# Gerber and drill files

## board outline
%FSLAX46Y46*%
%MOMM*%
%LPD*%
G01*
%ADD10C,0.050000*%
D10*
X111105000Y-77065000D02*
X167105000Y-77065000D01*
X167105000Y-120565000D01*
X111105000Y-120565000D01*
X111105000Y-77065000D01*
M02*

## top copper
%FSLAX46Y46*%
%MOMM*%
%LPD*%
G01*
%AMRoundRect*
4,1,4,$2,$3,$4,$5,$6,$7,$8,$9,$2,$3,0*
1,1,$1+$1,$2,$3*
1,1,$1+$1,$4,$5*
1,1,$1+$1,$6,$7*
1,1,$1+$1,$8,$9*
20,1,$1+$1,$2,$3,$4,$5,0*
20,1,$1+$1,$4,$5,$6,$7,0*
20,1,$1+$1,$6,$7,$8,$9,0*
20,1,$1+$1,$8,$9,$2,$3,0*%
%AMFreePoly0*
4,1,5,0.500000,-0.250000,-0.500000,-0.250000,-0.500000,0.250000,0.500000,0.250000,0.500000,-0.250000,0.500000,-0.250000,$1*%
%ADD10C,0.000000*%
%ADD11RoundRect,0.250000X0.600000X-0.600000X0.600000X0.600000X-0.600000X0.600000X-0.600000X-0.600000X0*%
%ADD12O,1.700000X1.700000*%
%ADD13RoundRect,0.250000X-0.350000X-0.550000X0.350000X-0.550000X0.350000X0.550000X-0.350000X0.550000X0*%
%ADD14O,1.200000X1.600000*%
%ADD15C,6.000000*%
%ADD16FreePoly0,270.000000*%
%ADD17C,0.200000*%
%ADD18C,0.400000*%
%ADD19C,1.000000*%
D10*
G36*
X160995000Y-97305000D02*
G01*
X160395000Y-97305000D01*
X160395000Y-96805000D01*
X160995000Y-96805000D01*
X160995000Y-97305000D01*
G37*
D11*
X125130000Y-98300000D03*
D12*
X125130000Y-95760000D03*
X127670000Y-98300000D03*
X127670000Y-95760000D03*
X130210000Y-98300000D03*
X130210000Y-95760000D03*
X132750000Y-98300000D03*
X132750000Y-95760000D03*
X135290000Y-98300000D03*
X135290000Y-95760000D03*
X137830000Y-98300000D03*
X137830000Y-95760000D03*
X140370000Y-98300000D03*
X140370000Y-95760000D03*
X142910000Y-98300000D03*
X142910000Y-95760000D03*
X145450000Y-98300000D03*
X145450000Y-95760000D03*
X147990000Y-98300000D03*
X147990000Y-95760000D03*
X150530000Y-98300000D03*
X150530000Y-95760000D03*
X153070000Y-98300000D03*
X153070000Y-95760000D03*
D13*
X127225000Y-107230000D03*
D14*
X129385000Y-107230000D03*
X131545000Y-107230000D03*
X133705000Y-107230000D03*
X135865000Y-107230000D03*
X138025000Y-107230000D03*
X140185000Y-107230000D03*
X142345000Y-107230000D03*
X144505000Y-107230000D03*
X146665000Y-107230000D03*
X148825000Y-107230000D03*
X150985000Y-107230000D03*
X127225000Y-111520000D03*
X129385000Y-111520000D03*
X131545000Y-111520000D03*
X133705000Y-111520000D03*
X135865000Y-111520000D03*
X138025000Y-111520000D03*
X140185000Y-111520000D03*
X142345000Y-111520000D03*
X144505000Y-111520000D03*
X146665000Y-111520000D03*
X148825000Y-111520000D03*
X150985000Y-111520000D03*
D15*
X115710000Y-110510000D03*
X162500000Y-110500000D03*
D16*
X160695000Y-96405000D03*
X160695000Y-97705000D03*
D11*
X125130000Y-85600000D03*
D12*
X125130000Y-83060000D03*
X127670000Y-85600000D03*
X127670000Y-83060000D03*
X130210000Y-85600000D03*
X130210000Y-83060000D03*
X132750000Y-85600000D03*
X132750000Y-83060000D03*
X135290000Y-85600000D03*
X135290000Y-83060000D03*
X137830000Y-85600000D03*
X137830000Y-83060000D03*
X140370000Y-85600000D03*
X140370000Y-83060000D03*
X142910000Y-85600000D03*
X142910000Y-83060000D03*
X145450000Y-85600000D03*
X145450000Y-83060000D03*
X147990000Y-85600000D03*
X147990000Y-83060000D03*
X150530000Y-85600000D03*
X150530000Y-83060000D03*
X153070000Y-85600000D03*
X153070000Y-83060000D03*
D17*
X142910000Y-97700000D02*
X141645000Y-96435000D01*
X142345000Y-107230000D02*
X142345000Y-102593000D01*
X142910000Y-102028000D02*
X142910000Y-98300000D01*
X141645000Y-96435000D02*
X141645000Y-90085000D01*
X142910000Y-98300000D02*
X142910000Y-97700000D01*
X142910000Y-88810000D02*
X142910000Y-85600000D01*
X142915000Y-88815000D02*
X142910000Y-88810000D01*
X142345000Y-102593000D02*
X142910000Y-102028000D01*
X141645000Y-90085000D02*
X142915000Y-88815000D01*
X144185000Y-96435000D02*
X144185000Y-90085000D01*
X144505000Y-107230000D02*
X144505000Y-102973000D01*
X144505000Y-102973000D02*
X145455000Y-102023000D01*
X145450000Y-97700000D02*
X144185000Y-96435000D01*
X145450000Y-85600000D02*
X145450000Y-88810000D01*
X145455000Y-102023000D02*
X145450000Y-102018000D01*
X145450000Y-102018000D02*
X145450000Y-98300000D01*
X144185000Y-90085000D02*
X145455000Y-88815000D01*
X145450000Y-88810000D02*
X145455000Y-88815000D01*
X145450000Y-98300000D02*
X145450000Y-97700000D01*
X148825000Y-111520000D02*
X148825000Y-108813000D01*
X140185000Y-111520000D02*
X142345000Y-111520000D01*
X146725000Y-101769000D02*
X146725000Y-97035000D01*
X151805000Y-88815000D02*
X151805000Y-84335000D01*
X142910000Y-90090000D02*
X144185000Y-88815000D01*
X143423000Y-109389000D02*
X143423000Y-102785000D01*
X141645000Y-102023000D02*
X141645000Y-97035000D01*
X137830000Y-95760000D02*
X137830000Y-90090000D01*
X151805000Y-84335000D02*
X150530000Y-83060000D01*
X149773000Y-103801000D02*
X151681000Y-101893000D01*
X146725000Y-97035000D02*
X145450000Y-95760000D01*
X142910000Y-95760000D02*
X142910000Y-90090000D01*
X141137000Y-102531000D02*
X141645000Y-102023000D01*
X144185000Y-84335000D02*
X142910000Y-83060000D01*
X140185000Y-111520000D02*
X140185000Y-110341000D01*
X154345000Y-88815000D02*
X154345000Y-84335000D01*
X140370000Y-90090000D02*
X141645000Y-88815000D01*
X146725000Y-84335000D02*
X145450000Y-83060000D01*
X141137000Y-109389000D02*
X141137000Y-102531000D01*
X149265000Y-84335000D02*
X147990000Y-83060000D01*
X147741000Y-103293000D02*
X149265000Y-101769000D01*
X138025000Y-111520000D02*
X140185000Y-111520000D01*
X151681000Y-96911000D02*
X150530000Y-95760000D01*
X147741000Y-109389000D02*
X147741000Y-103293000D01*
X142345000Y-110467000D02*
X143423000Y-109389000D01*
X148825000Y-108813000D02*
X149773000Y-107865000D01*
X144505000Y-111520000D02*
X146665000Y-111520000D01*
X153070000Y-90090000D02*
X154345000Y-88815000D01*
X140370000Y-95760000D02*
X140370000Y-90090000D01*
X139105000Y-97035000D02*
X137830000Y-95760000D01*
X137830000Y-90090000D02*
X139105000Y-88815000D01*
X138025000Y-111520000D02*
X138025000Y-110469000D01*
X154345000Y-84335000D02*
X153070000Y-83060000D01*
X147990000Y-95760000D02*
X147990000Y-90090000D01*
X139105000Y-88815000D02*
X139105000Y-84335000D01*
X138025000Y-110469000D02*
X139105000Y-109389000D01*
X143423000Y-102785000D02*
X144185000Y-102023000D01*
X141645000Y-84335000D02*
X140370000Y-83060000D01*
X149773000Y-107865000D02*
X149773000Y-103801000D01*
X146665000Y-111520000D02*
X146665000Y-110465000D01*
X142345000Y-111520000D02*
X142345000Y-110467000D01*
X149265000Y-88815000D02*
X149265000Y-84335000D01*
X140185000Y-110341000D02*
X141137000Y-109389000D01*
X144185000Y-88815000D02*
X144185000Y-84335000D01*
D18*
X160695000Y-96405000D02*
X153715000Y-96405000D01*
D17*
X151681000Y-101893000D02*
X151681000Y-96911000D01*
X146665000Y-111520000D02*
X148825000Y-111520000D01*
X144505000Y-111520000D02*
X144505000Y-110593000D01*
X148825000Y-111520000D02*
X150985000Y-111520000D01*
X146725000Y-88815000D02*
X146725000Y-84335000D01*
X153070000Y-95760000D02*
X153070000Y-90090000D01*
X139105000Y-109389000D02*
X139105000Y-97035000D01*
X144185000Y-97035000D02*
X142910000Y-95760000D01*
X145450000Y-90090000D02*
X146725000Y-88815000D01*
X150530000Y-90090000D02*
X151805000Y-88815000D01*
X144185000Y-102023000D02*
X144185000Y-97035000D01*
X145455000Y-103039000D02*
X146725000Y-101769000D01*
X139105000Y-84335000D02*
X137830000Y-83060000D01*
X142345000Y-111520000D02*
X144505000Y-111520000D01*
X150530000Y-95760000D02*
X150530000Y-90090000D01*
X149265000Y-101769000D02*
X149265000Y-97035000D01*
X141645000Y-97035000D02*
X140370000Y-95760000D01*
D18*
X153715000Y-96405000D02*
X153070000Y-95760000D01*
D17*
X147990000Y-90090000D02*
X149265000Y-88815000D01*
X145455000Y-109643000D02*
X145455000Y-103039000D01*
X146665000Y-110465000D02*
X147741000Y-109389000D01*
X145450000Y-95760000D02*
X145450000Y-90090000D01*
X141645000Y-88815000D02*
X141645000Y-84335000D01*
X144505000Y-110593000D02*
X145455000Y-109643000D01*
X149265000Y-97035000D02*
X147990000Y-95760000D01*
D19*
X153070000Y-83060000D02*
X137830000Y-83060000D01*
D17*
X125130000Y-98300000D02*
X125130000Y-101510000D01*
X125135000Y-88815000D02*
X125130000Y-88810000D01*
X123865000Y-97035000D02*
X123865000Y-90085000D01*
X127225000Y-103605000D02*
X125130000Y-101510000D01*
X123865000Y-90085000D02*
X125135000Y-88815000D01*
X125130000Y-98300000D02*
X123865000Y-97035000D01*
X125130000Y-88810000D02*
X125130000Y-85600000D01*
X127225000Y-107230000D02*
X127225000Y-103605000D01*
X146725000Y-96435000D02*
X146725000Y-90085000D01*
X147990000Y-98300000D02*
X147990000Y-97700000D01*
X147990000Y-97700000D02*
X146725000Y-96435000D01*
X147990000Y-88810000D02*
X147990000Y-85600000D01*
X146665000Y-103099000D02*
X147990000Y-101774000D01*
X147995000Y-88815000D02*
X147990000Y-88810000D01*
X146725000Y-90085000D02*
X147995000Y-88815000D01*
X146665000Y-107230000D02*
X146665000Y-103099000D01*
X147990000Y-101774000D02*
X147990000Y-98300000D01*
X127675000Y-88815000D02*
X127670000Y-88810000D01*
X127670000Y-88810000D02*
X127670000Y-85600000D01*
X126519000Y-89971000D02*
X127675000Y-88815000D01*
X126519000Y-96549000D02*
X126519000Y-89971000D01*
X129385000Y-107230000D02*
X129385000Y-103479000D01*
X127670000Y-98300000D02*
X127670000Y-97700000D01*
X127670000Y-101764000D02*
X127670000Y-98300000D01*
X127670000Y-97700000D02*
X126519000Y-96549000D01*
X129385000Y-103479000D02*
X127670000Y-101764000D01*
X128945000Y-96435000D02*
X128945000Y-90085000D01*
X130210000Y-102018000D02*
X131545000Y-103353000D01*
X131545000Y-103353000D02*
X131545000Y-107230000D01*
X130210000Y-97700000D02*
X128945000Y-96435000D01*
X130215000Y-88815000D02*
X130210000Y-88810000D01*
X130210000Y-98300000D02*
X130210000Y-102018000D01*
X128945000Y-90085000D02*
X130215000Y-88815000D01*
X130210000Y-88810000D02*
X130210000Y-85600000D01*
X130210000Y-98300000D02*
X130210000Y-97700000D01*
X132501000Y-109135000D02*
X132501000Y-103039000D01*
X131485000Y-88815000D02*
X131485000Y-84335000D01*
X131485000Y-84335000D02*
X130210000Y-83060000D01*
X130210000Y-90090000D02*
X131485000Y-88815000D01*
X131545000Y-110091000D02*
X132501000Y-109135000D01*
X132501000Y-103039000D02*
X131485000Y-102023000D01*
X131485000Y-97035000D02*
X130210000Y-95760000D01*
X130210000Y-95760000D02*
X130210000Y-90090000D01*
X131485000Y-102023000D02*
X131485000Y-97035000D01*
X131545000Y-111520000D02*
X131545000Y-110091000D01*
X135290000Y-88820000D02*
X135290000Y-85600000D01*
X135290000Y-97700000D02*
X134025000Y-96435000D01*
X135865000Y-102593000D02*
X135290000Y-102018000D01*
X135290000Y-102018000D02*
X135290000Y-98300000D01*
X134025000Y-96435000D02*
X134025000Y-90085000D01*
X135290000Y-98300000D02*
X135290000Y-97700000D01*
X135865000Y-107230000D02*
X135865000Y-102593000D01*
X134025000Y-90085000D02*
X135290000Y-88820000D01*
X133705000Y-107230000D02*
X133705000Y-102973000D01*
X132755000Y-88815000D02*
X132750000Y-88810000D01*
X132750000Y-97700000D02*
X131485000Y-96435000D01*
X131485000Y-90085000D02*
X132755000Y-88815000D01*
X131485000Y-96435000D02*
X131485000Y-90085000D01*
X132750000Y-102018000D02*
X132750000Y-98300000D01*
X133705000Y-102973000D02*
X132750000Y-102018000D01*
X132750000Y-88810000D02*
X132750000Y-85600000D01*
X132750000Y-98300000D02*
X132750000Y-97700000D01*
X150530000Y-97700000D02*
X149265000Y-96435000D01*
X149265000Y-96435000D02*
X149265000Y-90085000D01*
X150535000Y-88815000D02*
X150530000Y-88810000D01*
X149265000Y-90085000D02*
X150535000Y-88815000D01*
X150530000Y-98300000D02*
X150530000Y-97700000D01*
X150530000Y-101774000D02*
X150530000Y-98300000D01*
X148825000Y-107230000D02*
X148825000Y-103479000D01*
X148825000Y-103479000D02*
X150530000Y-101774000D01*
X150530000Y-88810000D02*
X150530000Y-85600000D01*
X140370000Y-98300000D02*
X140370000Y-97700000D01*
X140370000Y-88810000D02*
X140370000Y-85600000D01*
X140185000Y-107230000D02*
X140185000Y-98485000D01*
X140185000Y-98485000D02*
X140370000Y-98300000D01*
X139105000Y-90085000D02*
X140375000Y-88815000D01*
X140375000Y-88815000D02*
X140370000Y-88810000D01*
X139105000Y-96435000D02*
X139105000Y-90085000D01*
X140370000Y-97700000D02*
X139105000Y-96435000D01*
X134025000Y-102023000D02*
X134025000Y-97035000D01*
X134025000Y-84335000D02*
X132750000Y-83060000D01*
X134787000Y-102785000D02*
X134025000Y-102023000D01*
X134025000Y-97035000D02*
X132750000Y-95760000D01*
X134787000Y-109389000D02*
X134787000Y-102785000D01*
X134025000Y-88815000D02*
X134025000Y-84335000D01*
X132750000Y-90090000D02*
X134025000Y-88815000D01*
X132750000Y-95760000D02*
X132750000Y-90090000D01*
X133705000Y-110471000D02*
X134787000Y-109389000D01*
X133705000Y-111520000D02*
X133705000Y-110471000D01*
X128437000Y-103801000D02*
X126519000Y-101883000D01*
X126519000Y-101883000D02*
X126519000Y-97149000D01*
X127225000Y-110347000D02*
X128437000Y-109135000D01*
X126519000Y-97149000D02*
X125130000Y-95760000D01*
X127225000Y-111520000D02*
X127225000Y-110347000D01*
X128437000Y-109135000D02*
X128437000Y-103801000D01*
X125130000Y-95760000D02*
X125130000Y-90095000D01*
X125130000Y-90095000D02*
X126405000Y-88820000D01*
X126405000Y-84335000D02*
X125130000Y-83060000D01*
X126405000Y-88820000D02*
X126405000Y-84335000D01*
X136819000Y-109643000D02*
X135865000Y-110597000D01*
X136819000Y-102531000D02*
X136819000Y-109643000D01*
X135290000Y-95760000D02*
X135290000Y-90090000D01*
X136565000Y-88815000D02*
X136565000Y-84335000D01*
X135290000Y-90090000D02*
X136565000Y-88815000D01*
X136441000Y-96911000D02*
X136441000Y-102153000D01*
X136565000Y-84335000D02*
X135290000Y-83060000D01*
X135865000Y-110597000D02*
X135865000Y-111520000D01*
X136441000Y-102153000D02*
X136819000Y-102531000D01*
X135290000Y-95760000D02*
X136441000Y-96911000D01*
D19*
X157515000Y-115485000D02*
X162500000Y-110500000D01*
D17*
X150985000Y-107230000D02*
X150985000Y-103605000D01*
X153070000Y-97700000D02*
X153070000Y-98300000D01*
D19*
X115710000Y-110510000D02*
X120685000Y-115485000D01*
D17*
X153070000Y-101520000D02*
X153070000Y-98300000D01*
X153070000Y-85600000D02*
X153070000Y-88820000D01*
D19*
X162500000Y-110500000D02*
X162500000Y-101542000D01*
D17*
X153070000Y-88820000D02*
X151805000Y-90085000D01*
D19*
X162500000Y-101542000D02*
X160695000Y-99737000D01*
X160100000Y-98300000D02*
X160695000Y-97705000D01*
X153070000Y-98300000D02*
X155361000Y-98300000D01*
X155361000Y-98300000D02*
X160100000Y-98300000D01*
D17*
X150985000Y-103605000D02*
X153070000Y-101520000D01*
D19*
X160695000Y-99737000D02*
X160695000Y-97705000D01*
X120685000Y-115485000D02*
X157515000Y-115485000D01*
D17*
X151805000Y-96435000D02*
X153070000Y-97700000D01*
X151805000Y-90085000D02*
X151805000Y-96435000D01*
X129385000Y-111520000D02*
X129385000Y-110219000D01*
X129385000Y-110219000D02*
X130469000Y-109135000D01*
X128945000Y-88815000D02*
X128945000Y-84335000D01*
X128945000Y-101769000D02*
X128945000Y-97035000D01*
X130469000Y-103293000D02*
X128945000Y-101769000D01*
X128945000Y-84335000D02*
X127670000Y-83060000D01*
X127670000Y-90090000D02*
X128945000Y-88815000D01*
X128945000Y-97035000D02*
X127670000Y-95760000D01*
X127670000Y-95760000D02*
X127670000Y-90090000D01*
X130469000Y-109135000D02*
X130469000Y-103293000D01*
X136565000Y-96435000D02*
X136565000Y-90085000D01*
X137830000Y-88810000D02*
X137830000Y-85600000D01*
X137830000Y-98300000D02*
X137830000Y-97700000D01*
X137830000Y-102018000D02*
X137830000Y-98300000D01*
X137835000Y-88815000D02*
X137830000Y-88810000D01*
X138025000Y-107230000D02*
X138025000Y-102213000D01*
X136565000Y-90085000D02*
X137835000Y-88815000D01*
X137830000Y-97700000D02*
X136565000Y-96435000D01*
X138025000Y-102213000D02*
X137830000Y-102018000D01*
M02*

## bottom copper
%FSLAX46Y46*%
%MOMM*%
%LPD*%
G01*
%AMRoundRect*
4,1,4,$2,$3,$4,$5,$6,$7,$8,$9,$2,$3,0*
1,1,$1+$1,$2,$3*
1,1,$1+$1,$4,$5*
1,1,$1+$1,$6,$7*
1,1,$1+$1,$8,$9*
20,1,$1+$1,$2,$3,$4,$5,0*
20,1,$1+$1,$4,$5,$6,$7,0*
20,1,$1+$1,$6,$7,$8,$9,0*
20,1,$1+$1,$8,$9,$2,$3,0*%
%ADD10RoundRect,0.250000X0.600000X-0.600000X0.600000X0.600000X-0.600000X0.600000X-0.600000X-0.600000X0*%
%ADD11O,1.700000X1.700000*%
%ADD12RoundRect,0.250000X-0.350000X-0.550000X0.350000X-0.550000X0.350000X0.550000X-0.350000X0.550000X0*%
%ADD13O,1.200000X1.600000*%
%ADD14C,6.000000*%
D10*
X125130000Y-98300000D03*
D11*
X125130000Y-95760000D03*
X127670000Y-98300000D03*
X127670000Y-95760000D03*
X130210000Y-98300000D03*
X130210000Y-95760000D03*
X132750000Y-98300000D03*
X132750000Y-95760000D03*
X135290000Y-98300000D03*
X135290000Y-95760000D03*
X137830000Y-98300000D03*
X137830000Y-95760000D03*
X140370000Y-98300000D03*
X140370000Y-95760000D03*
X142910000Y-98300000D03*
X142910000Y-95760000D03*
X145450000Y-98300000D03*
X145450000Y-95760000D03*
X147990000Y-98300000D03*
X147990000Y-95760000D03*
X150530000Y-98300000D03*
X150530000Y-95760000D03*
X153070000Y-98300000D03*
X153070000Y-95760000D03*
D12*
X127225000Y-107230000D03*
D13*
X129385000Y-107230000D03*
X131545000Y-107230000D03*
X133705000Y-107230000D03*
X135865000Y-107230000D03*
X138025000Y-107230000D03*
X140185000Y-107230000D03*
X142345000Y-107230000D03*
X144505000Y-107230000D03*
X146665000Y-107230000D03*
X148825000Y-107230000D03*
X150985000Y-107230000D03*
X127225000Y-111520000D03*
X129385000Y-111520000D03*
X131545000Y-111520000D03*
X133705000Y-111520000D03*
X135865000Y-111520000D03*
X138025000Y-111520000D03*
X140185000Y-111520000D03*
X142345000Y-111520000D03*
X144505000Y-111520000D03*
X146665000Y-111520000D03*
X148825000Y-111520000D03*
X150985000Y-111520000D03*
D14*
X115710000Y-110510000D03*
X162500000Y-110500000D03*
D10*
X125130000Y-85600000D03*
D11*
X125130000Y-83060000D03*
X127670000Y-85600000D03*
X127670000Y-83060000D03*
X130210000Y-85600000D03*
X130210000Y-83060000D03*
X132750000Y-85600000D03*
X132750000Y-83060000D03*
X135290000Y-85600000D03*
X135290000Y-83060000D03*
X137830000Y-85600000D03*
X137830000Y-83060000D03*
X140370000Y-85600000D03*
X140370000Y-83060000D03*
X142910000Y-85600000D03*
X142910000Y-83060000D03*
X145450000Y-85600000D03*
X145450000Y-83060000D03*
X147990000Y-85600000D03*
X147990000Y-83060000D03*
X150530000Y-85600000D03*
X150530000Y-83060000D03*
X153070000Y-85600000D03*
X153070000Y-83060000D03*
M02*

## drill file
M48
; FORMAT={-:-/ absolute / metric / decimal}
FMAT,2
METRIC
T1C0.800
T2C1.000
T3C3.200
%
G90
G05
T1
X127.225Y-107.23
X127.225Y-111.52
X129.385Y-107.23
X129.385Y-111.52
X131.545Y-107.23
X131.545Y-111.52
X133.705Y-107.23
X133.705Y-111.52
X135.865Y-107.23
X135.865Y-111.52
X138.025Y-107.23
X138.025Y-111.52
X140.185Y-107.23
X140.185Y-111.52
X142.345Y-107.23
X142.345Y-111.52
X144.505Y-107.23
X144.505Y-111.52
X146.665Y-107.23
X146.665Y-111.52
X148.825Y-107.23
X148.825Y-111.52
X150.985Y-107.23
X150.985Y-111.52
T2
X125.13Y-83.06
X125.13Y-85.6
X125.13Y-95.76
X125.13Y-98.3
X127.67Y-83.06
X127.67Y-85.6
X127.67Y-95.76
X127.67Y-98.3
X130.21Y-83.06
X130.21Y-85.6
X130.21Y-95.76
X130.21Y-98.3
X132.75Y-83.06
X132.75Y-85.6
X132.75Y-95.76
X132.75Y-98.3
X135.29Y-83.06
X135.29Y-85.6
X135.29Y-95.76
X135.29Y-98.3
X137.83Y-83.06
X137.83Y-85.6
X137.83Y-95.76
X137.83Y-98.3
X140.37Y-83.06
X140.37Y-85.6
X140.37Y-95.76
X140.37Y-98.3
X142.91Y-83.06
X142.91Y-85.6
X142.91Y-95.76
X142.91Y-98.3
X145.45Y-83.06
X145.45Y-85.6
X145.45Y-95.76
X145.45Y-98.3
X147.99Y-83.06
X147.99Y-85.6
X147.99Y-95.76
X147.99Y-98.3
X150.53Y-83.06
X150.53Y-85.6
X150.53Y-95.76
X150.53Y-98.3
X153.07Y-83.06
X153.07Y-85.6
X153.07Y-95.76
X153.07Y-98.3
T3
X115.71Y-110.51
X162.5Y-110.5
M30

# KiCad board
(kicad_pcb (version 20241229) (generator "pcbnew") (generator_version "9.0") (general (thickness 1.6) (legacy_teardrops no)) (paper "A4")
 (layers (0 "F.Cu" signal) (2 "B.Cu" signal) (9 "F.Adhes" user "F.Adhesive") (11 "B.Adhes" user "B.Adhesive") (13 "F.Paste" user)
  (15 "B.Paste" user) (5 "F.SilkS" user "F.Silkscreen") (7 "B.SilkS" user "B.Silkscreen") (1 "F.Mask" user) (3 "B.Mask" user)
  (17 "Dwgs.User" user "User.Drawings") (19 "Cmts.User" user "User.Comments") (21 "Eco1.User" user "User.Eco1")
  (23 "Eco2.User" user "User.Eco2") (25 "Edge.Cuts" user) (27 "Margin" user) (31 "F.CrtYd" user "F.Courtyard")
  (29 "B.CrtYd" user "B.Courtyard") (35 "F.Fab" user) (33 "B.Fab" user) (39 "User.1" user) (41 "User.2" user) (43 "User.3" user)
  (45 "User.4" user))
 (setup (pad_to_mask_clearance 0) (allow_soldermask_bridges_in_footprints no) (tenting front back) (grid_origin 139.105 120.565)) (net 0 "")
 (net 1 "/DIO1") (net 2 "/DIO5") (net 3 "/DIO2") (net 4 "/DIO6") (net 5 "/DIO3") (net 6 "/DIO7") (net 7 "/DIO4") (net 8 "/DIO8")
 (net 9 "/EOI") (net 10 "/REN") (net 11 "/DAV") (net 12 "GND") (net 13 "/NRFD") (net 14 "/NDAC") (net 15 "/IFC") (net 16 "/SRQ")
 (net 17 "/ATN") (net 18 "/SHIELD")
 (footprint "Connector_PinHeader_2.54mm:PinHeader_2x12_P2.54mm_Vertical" (layer "F.Cu") (at 125.13 98.3 90)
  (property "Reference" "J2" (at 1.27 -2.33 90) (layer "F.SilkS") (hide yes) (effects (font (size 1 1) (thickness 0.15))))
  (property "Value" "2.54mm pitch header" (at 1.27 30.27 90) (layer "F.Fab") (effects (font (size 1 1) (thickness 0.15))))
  (pad "1" thru_hole roundrect (at 0 0 90) (size 1.7 1.7) (drill 1) (layers "*.Cu" "*.Mask") (remove_unused_layers no)
   (roundrect_rratio 0.1470588235) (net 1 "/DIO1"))
  (pad "2" thru_hole oval (at 2.54 0 90) (size 1.7 1.7) (drill 1) (layers "*.Cu" "*.Mask") (remove_unused_layers no) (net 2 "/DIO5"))
  (pad "3" thru_hole oval (at 0 2.54 90) (size 1.7 1.7) (drill 1) (layers "*.Cu" "*.Mask") (remove_unused_layers no) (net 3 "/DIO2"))
  (pad "4" thru_hole oval (at 2.54 2.54 90) (size 1.7 1.7) (drill 1) (layers "*.Cu" "*.Mask") (remove_unused_layers no) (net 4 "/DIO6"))
  (pad "5" thru_hole oval (at 0 5.08 90) (size 1.7 1.7) (drill 1) (layers "*.Cu" "*.Mask") (remove_unused_layers no) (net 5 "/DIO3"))
  (pad "6" thru_hole oval (at 2.54 5.08 90) (size 1.7 1.7) (drill 1) (layers "*.Cu" "*.Mask") (remove_unused_layers no) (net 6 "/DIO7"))
  (pad "7" thru_hole oval (at 0 7.62 90) (size 1.7 1.7) (drill 1) (layers "*.Cu" "*.Mask") (remove_unused_layers no) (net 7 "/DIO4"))
  (pad "8" thru_hole oval (at 2.54 7.62 90) (size 1.7 1.7) (drill 1) (layers "*.Cu" "*.Mask") (remove_unused_layers no) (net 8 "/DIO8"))
  (pad "9" thru_hole oval (at 0 10.16 90) (size 1.7 1.7) (drill 1) (layers "*.Cu" "*.Mask") (remove_unused_layers no) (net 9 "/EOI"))
  (pad "10" thru_hole oval (at 2.54 10.16 90) (size 1.7 1.7) (drill 1) (layers "*.Cu" "*.Mask") (remove_unused_layers no) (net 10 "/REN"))
  (pad "11" thru_hole oval (at 0 12.7 90) (size 1.7 1.7) (drill 1) (layers "*.Cu" "*.Mask") (remove_unused_layers no) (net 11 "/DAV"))
  (pad "12" thru_hole oval (at 2.54 12.7 90) (size 1.7 1.7) (drill 1) (layers "*.Cu" "*.Mask") (remove_unused_layers no) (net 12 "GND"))
  (pad "13" thru_hole oval (at 0 15.24 90) (size 1.7 1.7) (drill 1) (layers "*.Cu" "*.Mask") (remove_unused_layers no) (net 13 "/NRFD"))
  (pad "14" thru_hole oval (at 2.54 15.24 90) (size 1.7 1.7) (drill 1) (layers "*.Cu" "*.Mask") (remove_unused_layers no) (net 12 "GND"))
  (pad "15" thru_hole oval (at 0 17.78 90) (size 1.7 1.7) (drill 1) (layers "*.Cu" "*.Mask") (remove_unused_layers no) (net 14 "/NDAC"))
  (pad "16" thru_hole oval (at 2.54 17.78 90) (size 1.7 1.7) (drill 1) (layers "*.Cu" "*.Mask") (remove_unused_layers no) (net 12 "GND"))
  (pad "17" thru_hole oval (at 0 20.32 90) (size 1.7 1.7) (drill 1) (layers "*.Cu" "*.Mask") (remove_unused_layers no) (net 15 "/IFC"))
  (pad "18" thru_hole oval (at 2.54 20.32 90) (size 1.7 1.7) (drill 1) (layers "*.Cu" "*.Mask") (remove_unused_layers no) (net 12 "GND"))
  (pad "19" thru_hole oval (at 0 22.86 90) (size 1.7 1.7) (drill 1) (layers "*.Cu" "*.Mask") (remove_unused_layers no) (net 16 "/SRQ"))
  (pad "20" thru_hole oval (at 2.54 22.86 90) (size 1.7 1.7) (drill 1) (layers "*.Cu" "*.Mask") (remove_unused_layers no) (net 12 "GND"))
  (pad "21" thru_hole oval (at 0 25.4 90) (size 1.7 1.7) (drill 1) (layers "*.Cu" "*.Mask") (remove_unused_layers no) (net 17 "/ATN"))
  (pad "22" thru_hole oval (at 2.54 25.4 90) (size 1.7 1.7) (drill 1) (layers "*.Cu" "*.Mask") (remove_unused_layers no) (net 12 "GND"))
  (pad "23" thru_hole oval (at 0 27.94 90) (size 1.7 1.7) (drill 1) (layers "*.Cu" "*.Mask") (remove_unused_layers no) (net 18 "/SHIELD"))
  (pad "24" thru_hole oval (at 2.54 27.94 90) (size 1.7 1.7) (drill 1) (layers "*.Cu" "*.Mask") (remove_unused_layers no) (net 12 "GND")))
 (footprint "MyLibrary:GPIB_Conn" (layer "F.Cu") (at 127.225 107.23)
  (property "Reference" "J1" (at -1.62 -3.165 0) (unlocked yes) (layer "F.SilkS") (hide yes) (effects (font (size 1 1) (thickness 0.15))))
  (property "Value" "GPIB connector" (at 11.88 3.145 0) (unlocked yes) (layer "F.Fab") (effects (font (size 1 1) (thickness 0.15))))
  (pad "1" thru_hole roundrect (at 0 0) (size 1.2 1.6) (drill 0.8) (layers "*.Cu" "*.Mask") (remove_unused_layers no)
   (roundrect_rratio 0.2083333333) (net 1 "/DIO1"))
  (pad "2" thru_hole oval (at 2.16 0) (size 1.2 1.6) (drill 0.8) (layers "*.Cu" "*.Mask") (remove_unused_layers no) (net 3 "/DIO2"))
  (pad "3" thru_hole oval (at 4.32 0) (size 1.2 1.6) (drill 0.8) (layers "*.Cu" "*.Mask") (remove_unused_layers no) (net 5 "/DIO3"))
  (pad "4" thru_hole oval (at 6.48 0) (size 1.2 1.6) (drill 0.8) (layers "*.Cu" "*.Mask") (remove_unused_layers no) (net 7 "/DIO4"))
  (pad "5" thru_hole oval (at 8.64 0) (size 1.2 1.6) (drill 0.8) (layers "*.Cu" "*.Mask") (remove_unused_layers no) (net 9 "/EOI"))
  (pad "6" thru_hole oval (at 10.8 0) (size 1.2 1.6) (drill 0.8) (layers "*.Cu" "*.Mask") (remove_unused_layers no) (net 11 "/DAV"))
  (pad "7" thru_hole oval (at 12.96 0) (size 1.2 1.6) (drill 0.8) (layers "*.Cu" "*.Mask") (remove_unused_layers no) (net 13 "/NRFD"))
  (pad "8" thru_hole oval (at 15.12 0) (size 1.2 1.6) (drill 0.8) (layers "*.Cu" "*.Mask") (remove_unused_layers no) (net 14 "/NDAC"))
  (pad "9" thru_hole oval (at 17.28 0) (size 1.2 1.6) (drill 0.8) (layers "*.Cu" "*.Mask") (remove_unused_layers no) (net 15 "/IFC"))
  (pad "10" thru_hole oval (at 19.44 0) (size 1.2 1.6) (drill 0.8) (layers "*.Cu" "*.Mask") (remove_unused_layers no) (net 16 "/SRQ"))
  (pad "11" thru_hole oval (at 21.6 0) (size 1.2 1.6) (drill 0.8) (layers "*.Cu" "*.Mask") (remove_unused_layers no) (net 17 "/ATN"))
  (pad "12" thru_hole oval (at 23.76 0) (size 1.2 1.6) (drill 0.8) (layers "*.Cu" "*.Mask") (remove_unused_layers no) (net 18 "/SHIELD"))
  (pad "13" thru_hole oval (at 0 4.29) (size 1.2 1.6) (drill 0.8) (layers "*.Cu" "*.Mask") (remove_unused_layers no) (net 2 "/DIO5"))
  (pad "14" thru_hole oval (at 2.16 4.29) (size 1.2 1.6) (drill 0.8) (layers "*.Cu" "*.Mask") (remove_unused_layers no) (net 4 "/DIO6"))
  (pad "15" thru_hole oval (at 4.32 4.29) (size 1.2 1.6) (drill 0.8) (layers "*.Cu" "*.Mask") (remove_unused_layers no) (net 6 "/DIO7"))
  (pad "16" thru_hole oval (at 6.48 4.29) (size 1.2 1.6) (drill 0.8) (layers "*.Cu" "*.Mask") (remove_unused_layers no) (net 8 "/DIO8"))
  (pad "17" thru_hole oval (at 8.64 4.29) (size 1.2 1.6) (drill 0.8) (layers "*.Cu" "*.Mask") (remove_unused_layers no) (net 10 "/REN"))
  (pad "18" thru_hole oval (at 10.8 4.29) (size 1.2 1.6) (drill 0.8) (layers "*.Cu" "*.Mask") (remove_unused_layers no) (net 12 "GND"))
  (pad "19" thru_hole oval (at 12.96 4.29) (size 1.2 1.6) (drill 0.8) (layers "*.Cu" "*.Mask") (remove_unused_layers no) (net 12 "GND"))
  (pad "20" thru_hole oval (at 15.12 4.29) (size 1.2 1.6) (drill 0.8) (layers "*.Cu" "*.Mask") (remove_unused_layers no) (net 12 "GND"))
  (pad "21" thru_hole oval (at 17.28 4.29) (size 1.2 1.6) (drill 0.8) (layers "*.Cu" "*.Mask") (remove_unused_layers no) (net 12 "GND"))
  (pad "22" thru_hole oval (at 19.44 4.29) (size 1.2 1.6) (drill 0.8) (layers "*.Cu" "*.Mask") (remove_unused_layers no) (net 12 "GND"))
  (pad "23" thru_hole oval (at 21.6 4.29) (size 1.2 1.6) (drill 0.8) (layers "*.Cu" "*.Mask") (remove_unused_layers no) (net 12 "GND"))
  (pad "24" thru_hole oval (at 23.76 4.29) (size 1.2 1.6) (drill 0.8) (layers "*.Cu" "*.Mask") (remove_unused_layers no) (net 12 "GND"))
  (pad "MP" thru_hole circle (at -11.515 3.28) (size 6 6) (drill 3.2) (layers "*.Cu" "*.Mask") (remove_unused_layers no) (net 18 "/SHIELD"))
  (pad "MP" thru_hole circle (at 35.275 3.27) (size 6 6) (drill 3.2) (layers "*.Cu" "*.Mask") (remove_unused_layers no) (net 18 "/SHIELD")))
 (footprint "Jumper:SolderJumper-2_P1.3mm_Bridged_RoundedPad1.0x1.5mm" (layer "F.Cu") (at 160.695 97.055 -90)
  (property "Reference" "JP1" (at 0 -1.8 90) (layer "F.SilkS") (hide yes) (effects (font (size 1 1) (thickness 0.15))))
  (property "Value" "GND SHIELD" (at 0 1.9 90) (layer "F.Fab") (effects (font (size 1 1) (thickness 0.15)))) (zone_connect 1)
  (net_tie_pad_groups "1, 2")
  (fp_poly (pts (xy 0.25 -0.3) (xy -0.25 -0.3) (xy -0.25 0.3) (xy 0.25 0.3)) (stroke (width 0) (type solid)) (fill yes) (layer "F.Cu"))
  (pad "1" smd custom (at -0.65 0 270) (size 1 0.5) (layers "F.Cu" "F.Mask") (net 12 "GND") (zone_connect 2) (thermal_bridge_angle 45)
   (options (clearance outline) (anchor rect)) (primitives))
  (pad "2" smd custom (at 0.65 0 270) (size 1 0.5) (layers "F.Cu" "F.Mask") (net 18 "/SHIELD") (zone_connect 2) (thermal_bridge_angle 45)
   (options (clearance outline) (anchor rect)) (primitives)))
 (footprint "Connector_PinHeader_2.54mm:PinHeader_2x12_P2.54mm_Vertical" (layer "F.Cu") (at 125.13 85.6 90)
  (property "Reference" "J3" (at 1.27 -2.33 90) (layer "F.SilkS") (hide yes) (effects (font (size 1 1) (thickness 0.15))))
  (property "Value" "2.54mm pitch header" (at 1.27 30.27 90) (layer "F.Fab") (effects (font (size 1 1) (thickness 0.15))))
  (pad "1" thru_hole roundrect (at 0 0 90) (size 1.7 1.7) (drill 1) (layers "*.Cu" "*.Mask") (remove_unused_layers no)
   (roundrect_rratio 0.1470588235) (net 1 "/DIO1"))
  (pad "2" thru_hole oval (at 2.54 0 90) (size 1.7 1.7) (drill 1) (layers "*.Cu" "*.Mask") (remove_unused_layers no) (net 2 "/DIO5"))
  (pad "3" thru_hole oval (at 0 2.54 90) (size 1.7 1.7) (drill 1) (layers "*.Cu" "*.Mask") (remove_unused_layers no) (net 3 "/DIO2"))
  (pad "4" thru_hole oval (at 2.54 2.54 90) (size 1.7 1.7) (drill 1) (layers "*.Cu" "*.Mask") (remove_unused_layers no) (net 4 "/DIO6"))
  (pad "5" thru_hole oval (at 0 5.08 90) (size 1.7 1.7) (drill 1) (layers "*.Cu" "*.Mask") (remove_unused_layers no) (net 5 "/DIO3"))
  (pad "6" thru_hole oval (at 2.54 5.08 90) (size 1.7 1.7) (drill 1) (layers "*.Cu" "*.Mask") (remove_unused_layers no) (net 6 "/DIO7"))
  (pad "7" thru_hole oval (at 0 7.62 90) (size 1.7 1.7) (drill 1) (layers "*.Cu" "*.Mask") (remove_unused_layers no) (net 7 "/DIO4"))
  (pad "8" thru_hole oval (at 2.54 7.62 90) (size 1.7 1.7) (drill 1) (layers "*.Cu" "*.Mask") (remove_unused_layers no) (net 8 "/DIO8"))
  (pad "9" thru_hole oval (at 0 10.16 90) (size 1.7 1.7) (drill 1) (layers "*.Cu" "*.Mask") (remove_unused_layers no) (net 9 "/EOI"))
  (pad "10" thru_hole oval (at 2.54 10.16 90) (size 1.7 1.7) (drill 1) (layers "*.Cu" "*.Mask") (remove_unused_layers no) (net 10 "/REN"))
  (pad "11" thru_hole oval (at 0 12.7 90) (size 1.7 1.7) (drill 1) (layers "*.Cu" "*.Mask") (remove_unused_layers no) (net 11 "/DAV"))
  (pad "12" thru_hole oval (at 2.54 12.7 90) (size 1.7 1.7) (drill 1) (layers "*.Cu" "*.Mask") (remove_unused_layers no) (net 12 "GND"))
  (pad "13" thru_hole oval (at 0 15.24 90) (size 1.7 1.7) (drill 1) (layers "*.Cu" "*.Mask") (remove_unused_layers no) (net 13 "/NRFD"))
  (pad "14" thru_hole oval (at 2.54 15.24 90) (size 1.7 1.7) (drill 1) (layers "*.Cu" "*.Mask") (remove_unused_layers no) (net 12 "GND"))
  (pad "15" thru_hole oval (at 0 17.78 90) (size 1.7 1.7) (drill 1) (layers "*.Cu" "*.Mask") (remove_unused_layers no) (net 14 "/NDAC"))
  (pad "16" thru_hole oval (at 2.54 17.78 90) (size 1.7 1.7) (drill 1) (layers "*.Cu" "*.Mask") (remove_unused_layers no) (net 12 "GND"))
  (pad "17" thru_hole oval (at 0 20.32 90) (size 1.7 1.7) (drill 1) (layers "*.Cu" "*.Mask") (remove_unused_layers no) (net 15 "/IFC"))
  (pad "18" thru_hole oval (at 2.54 20.32 90) (size 1.7 1.7) (drill 1) (layers "*.Cu" "*.Mask") (remove_unused_layers no) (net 12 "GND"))
  (pad "19" thru_hole oval (at 0 22.86 90) (size 1.7 1.7) (drill 1) (layers "*.Cu" "*.Mask") (remove_unused_layers no) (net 16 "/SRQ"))
  (pad "20" thru_hole oval (at 2.54 22.86 90) (size 1.7 1.7) (drill 1) (layers "*.Cu" "*.Mask") (remove_unused_layers no) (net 12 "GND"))
  (pad "21" thru_hole oval (at 0 25.4 90) (size 1.7 1.7) (drill 1) (layers "*.Cu" "*.Mask") (remove_unused_layers no) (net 17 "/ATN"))
  (pad "22" thru_hole oval (at 2.54 25.4 90) (size 1.7 1.7) (drill 1) (layers "*.Cu" "*.Mask") (remove_unused_layers no) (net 12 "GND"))
  (pad "23" thru_hole oval (at 0 27.94 90) (size 1.7 1.7) (drill 1) (layers "*.Cu" "*.Mask") (remove_unused_layers no) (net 18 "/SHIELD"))
  (pad "24" thru_hole oval (at 2.54 27.94 90) (size 1.7 1.7) (drill 1) (layers "*.Cu" "*.Mask") (remove_unused_layers no) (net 12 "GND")))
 (gr_rect (start 111.105 77.065) (end 167.105 120.565) (stroke (width 0.05) (type default)) (fill no) (layer "Edge.Cuts"))
 (segment (start 142.91 97.7) (end 141.645 96.435) (width 0.2) (layer "F.Cu") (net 14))
 (segment (start 142.345 107.23) (end 142.345 102.593) (width 0.2) (layer "F.Cu") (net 14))
 (segment (start 142.91 102.028) (end 142.91 98.3) (width 0.2) (layer "F.Cu") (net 14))
 (segment (start 141.645 96.435) (end 141.645 90.085) (width 0.2) (layer "F.Cu") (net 14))
 (segment (start 142.91 98.3) (end 142.91 97.7) (width 0.2) (layer "F.Cu") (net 14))
 (segment (start 142.91 88.81) (end 142.91 85.6) (width 0.2) (layer "F.Cu") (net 14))
 (segment (start 142.915 88.815) (end 142.91 88.81) (width 0.2) (layer "F.Cu") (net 14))
 (segment (start 142.345 102.593) (end 142.91 102.028) (width 0.2) (layer "F.Cu") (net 14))
 (segment (start 141.645 90.085) (end 142.915 88.815) (width 0.2) (layer "F.Cu") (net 14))
 (segment (start 144.185 96.435) (end 144.185 90.085) (width 0.2) (layer "F.Cu") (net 15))
 (segment (start 144.505 107.23) (end 144.505 102.973) (width 0.2) (layer "F.Cu") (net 15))
 (segment (start 144.505 102.973) (end 145.455 102.023) (width 0.2) (layer "F.Cu") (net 15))
 (segment (start 145.45 97.7) (end 144.185 96.435) (width 0.2) (layer "F.Cu") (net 15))
 (segment (start 145.45 85.6) (end 145.45 88.81) (width 0.2) (layer "F.Cu") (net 15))
 (segment (start 145.455 102.023) (end 145.45 102.018) (width 0.2) (layer "F.Cu") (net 15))
 (segment (start 145.45 102.018) (end 145.45 98.3) (width 0.2) (layer "F.Cu") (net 15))
 (segment (start 144.185 90.085) (end 145.455 88.815) (width 0.2) (layer "F.Cu") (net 15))
 (segment (start 145.45 88.81) (end 145.455 88.815) (width 0.2) (layer "F.Cu") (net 15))
 (segment (start 145.45 98.3) (end 145.45 97.7) (width 0.2) (layer "F.Cu") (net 15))
 (segment (start 148.825 111.52) (end 148.825 108.813) (width 0.2) (layer "F.Cu") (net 12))
 (segment (start 140.185 111.52) (end 142.345 111.52) (width 0.2) (layer "F.Cu") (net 12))
 (segment (start 146.725 101.769) (end 146.725 97.035) (width 0.2) (layer "F.Cu") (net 12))
 (segment (start 151.805 88.815) (end 151.805 84.335) (width 0.2) (layer "F.Cu") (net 12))
 (segment (start 142.91 90.09) (end 144.185 88.815) (width 0.2) (layer "F.Cu") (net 12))
 (segment (start 143.423 109.389) (end 143.423 102.785) (width 0.2) (layer "F.Cu") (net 12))
 (segment (start 141.645 102.023) (end 141.645 97.035) (width 0.2) (layer "F.Cu") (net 12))
 (segment (start 137.83 95.76) (end 137.83 90.09) (width 0.2) (layer "F.Cu") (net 12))
 (segment (start 151.805 84.335) (end 150.53 83.06) (width 0.2) (layer "F.Cu") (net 12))
 (segment (start 149.773 103.801) (end 151.681 101.893) (width 0.2) (layer "F.Cu") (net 12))
 (segment (start 146.725 97.035) (end 145.45 95.76) (width 0.2) (layer "F.Cu") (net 12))
 (segment (start 142.91 95.76) (end 142.91 90.09) (width 0.2) (layer "F.Cu") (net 12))
 (segment (start 141.137 102.531) (end 141.645 102.023) (width 0.2) (layer "F.Cu") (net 12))
 (segment (start 144.185 84.335) (end 142.91 83.06) (width 0.2) (layer "F.Cu") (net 12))
 (segment (start 140.185 111.52) (end 140.185 110.341) (width 0.2) (layer "F.Cu") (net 12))
 (segment (start 154.345 88.815) (end 154.345 84.335) (width 0.2) (layer "F.Cu") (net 12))
 (segment (start 140.37 90.09) (end 141.645 88.815) (width 0.2) (layer "F.Cu") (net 12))
 (segment (start 146.725 84.335) (end 145.45 83.06) (width 0.2) (layer "F.Cu") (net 12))
 (segment (start 141.137 109.389) (end 141.137 102.531) (width 0.2) (layer "F.Cu") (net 12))
 (segment (start 149.265 84.335) (end 147.99 83.06) (width 0.2) (layer "F.Cu") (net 12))
 (segment (start 147.741 103.293) (end 149.265 101.769) (width 0.2) (layer "F.Cu") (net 12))
 (segment (start 138.025 111.52) (end 140.185 111.52) (width 0.2) (layer "F.Cu") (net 12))
 (segment (start 151.681 96.911) (end 150.53 95.76) (width 0.2) (layer "F.Cu") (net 12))
 (segment (start 147.741 109.389) (end 147.741 103.293) (width 0.2) (layer "F.Cu") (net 12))
 (segment (start 142.345 110.467) (end 143.423 109.389) (width 0.2) (layer "F.Cu") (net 12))
 (segment (start 148.825 108.813) (end 149.773 107.865) (width 0.2) (layer "F.Cu") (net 12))
 (segment (start 144.505 111.52) (end 146.665 111.52) (width 0.2) (layer "F.Cu") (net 12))
 (segment (start 153.07 90.09) (end 154.345 88.815) (width 0.2) (layer "F.Cu") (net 12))
 (segment (start 140.37 95.76) (end 140.37 90.09) (width 0.2) (layer "F.Cu") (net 12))
 (segment (start 139.105 97.035) (end 137.83 95.76) (width 0.2) (layer "F.Cu") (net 12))
 (segment (start 137.83 90.09) (end 139.105 88.815) (width 0.2) (layer "F.Cu") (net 12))
 (segment (start 138.025 111.52) (end 138.025 110.469) (width 0.2) (layer "F.Cu") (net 12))
 (segment (start 154.345 84.335) (end 153.07 83.06) (width 0.2) (layer "F.Cu") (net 12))
 (segment (start 147.99 95.76) (end 147.99 90.09) (width 0.2) (layer "F.Cu") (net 12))
 (segment (start 139.105 88.815) (end 139.105 84.335) (width 0.2) (layer "F.Cu") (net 12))
 (segment (start 138.025 110.469) (end 139.105 109.389) (width 0.2) (layer "F.Cu") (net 12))
 (segment (start 143.423 102.785) (end 144.185 102.023) (width 0.2) (layer "F.Cu") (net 12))
 (segment (start 141.645 84.335) (end 140.37 83.06) (width 0.2) (layer "F.Cu") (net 12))
 (segment (start 149.773 107.865) (end 149.773 103.801) (width 0.2) (layer "F.Cu") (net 12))
 (segment (start 146.665 111.52) (end 146.665 110.465) (width 0.2) (layer "F.Cu") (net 12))
 (segment (start 142.345 111.52) (end 142.345 110.467) (width 0.2) (layer "F.Cu") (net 12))
 (segment (start 149.265 88.815) (end 149.265 84.335) (width 0.2) (layer "F.Cu") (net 12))
 (segment (start 140.185 110.341) (end 141.137 109.389) (width 0.2) (layer "F.Cu") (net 12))
 (segment (start 144.185 88.815) (end 144.185 84.335) (width 0.2) (layer "F.Cu") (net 12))
 (segment (start 160.695 96.405) (end 153.715 96.405) (width 0.4) (layer "F.Cu") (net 12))
 (segment (start 151.681 101.893) (end 151.681 96.911) (width 0.2) (layer "F.Cu") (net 12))
 (segment (start 146.665 111.52) (end 148.825 111.52) (width 0.2) (layer "F.Cu") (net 12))
 (segment (start 144.505 111.52) (end 144.505 110.593) (width 0.2) (layer "F.Cu") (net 12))
 (segment (start 148.825 111.52) (end 150.985 111.52) (width 0.2) (layer "F.Cu") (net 12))
 (segment (start 146.725 88.815) (end 146.725 84.335) (width 0.2) (layer "F.Cu") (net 12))
 (segment (start 153.07 95.76) (end 153.07 90.09) (width 0.2) (layer "F.Cu") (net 12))
 (segment (start 139.105 109.389) (end 139.105 97.035) (width 0.2) (layer "F.Cu") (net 12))
 (segment (start 144.185 97.035) (end 142.91 95.76) (width 0.2) (layer "F.Cu") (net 12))
 (segment (start 145.45 90.09) (end 146.725 88.815) (width 0.2) (layer "F.Cu") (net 12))
 (segment (start 150.53 90.09) (end 151.805 88.815) (width 0.2) (layer "F.Cu") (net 12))
 (segment (start 144.185 102.023) (end 144.185 97.035) (width 0.2) (layer "F.Cu") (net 12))
 (segment (start 145.455 103.039) (end 146.725 101.769) (width 0.2) (layer "F.Cu") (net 12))
 (segment (start 139.105 84.335) (end 137.83 83.06) (width 0.2) (layer "F.Cu") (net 12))
 (segment (start 142.345 111.52) (end 144.505 111.52) (width 0.2) (layer "F.Cu") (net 12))
 (segment (start 150.53 95.76) (end 150.53 90.09) (width 0.2) (layer "F.Cu") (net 12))
 (segment (start 149.265 101.769) (end 149.265 97.035) (width 0.2) (layer "F.Cu") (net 12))
 (segment (start 141.645 97.035) (end 140.37 95.76) (width 0.2) (layer "F.Cu") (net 12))
 (segment (start 153.715 96.405) (end 153.07 95.76) (width 0.4) (layer "F.Cu") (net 12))
 (segment (start 147.99 90.09) (end 149.265 88.815) (width 0.2) (layer "F.Cu") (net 12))
 (segment (start 145.455 109.643) (end 145.455 103.039) (width 0.2) (layer "F.Cu") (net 12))
 (segment (start 146.665 110.465) (end 147.741 109.389) (width 0.2) (layer "F.Cu") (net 12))
 (segment (start 145.45 95.76) (end 145.45 90.09) (width 0.2) (layer "F.Cu") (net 12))
 (segment (start 141.645 88.815) (end 141.645 84.335) (width 0.2) (layer "F.Cu") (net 12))
 (segment (start 144.505 110.593) (end 145.455 109.643) (width 0.2) (layer "F.Cu") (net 12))
 (segment (start 149.265 97.035) (end 147.99 95.76) (width 0.2) (layer "F.Cu") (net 12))
 (segment (start 153.07 83.06) (end 137.83 83.06) (width 1) (layer "F.Cu") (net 12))
 (segment (start 125.13 98.3) (end 125.13 101.51) (width 0.2) (layer "F.Cu") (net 1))
 (segment (start 125.135 88.815) (end 125.13 88.81) (width 0.2) (layer "F.Cu") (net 1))
 (segment (start 123.865 97.035) (end 123.865 90.085) (width 0.2) (layer "F.Cu") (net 1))
 (segment (start 127.225 103.605) (end 125.13 101.51) (width 0.2) (layer "F.Cu") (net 1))
 (segment (start 123.865 90.085) (end 125.135 88.815) (width 0.2) (layer "F.Cu") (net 1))
 (segment (start 125.13 98.3) (end 123.865 97.035) (width 0.2) (layer "F.Cu") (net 1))
 (segment (start 125.13 88.81) (end 125.13 85.6) (width 0.2) (layer "F.Cu") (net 1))
 (segment (start 127.225 107.23) (end 127.225 103.605) (width 0.2) (layer "F.Cu") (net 1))
 (segment (start 146.725 96.435) (end 146.725 90.085) (width 0.2) (layer "F.Cu") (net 16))
 (segment (start 147.99 98.3) (end 147.99 97.7) (width 0.2) (layer "F.Cu") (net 16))
 (segment (start 147.99 97.7) (end 146.725 96.435) (width 0.2) (layer "F.Cu") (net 16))
 (segment (start 147.99 88.81) (end 147.99 85.6) (width 0.2) (layer "F.Cu") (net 16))
 (segment (start 146.665 103.099) (end 147.99 101.774) (width 0.2) (layer "F.Cu") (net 16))
 (segment (start 147.995 88.815) (end 147.99 88.81) (width 0.2) (layer "F.Cu") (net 16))
 (segment (start 146.725 90.085) (end 147.995 88.815) (width 0.2) (layer "F.Cu") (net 16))
 (segment (start 146.665 107.23) (end 146.665 103.099) (width 0.2) (layer "F.Cu") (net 16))
 (segment (start 147.99 101.774) (end 147.99 98.3) (width 0.2) (layer "F.Cu") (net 16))
 (segment (start 127.675 88.815) (end 127.67 88.81) (width 0.2) (layer "F.Cu") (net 3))
 (segment (start 127.67 88.81) (end 127.67 85.6) (width 0.2) (layer "F.Cu") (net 3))
 (segment (start 126.519 89.971) (end 127.675 88.815) (width 0.2) (layer "F.Cu") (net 3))
 (segment (start 126.519 96.549) (end 126.519 89.971) (width 0.2) (layer "F.Cu") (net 3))
 (segment (start 129.385 107.23) (end 129.385 103.479) (width 0.2) (layer "F.Cu") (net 3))
 (segment (start 127.67 98.3) (end 127.67 97.7) (width 0.2) (layer "F.Cu") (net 3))
 (segment (start 127.67 101.764) (end 127.67 98.3) (width 0.2) (layer "F.Cu") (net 3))
 (segment (start 127.67 97.7) (end 126.519 96.549) (width 0.2) (layer "F.Cu") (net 3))
 (segment (start 129.385 103.479) (end 127.67 101.764) (width 0.2) (layer "F.Cu") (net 3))
 (segment (start 128.945 96.435) (end 128.945 90.085) (width 0.2) (layer "F.Cu") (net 5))
 (segment (start 130.21 102.018) (end 131.545 103.353) (width 0.2) (layer "F.Cu") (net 5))
 (segment (start 131.545 103.353) (end 131.545 107.23) (width 0.2) (layer "F.Cu") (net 5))
 (segment (start 130.21 97.7) (end 128.945 96.435) (width 0.2) (layer "F.Cu") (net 5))
 (segment (start 130.215 88.815) (end 130.21 88.81) (width 0.2) (layer "F.Cu") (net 5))
 (segment (start 130.21 98.3) (end 130.21 102.018) (width 0.2) (layer "F.Cu") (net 5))
 (segment (start 128.945 90.085) (end 130.215 88.815) (width 0.2) (layer "F.Cu") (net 5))
 (segment (start 130.21 88.81) (end 130.21 85.6) (width 0.2) (layer "F.Cu") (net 5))
 (segment (start 130.21 98.3) (end 130.21 97.7) (width 0.2) (layer "F.Cu") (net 5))
 (segment (start 132.501 109.135) (end 132.501 103.039) (width 0.2) (layer "F.Cu") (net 6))
 (segment (start 131.485 88.815) (end 131.485 84.335) (width 0.2) (layer "F.Cu") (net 6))
 (segment (start 131.485 84.335) (end 130.21 83.06) (width 0.2) (layer "F.Cu") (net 6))
 (segment (start 130.21 90.09) (end 131.485 88.815) (width 0.2) (layer "F.Cu") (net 6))
 (segment (start 131.545 110.091) (end 132.501 109.135) (width 0.2) (layer "F.Cu") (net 6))
 (segment (start 132.501 103.039) (end 131.485 102.023) (width 0.2) (layer "F.Cu") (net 6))
 (segment (start 131.485 97.035) (end 130.21 95.76) (width 0.2) (layer "F.Cu") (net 6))
 (segment (start 130.21 95.76) (end 130.21 90.09) (width 0.2) (layer "F.Cu") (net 6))
 (segment (start 131.485 102.023) (end 131.485 97.035) (width 0.2) (layer "F.Cu") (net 6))
 (segment (start 131.545 111.52) (end 131.545 110.091) (width 0.2) (layer "F.Cu") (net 6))
 (segment (start 135.29 88.82) (end 135.29 85.6) (width 0.2) (layer "F.Cu") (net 9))
 (segment (start 135.29 97.7) (end 134.025 96.435) (width 0.2) (layer "F.Cu") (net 9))
 (segment (start 135.865 102.593) (end 135.29 102.018) (width 0.2) (layer "F.Cu") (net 9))
 (segment (start 135.29 102.018) (end 135.29 98.3) (width 0.2) (layer "F.Cu") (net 9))
 (segment (start 134.025 96.435) (end 134.025 90.085) (width 0.2) (layer "F.Cu") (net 9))
 (segment (start 135.29 98.3) (end 135.29 97.7) (width 0.2) (layer "F.Cu") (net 9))
 (segment (start 135.865 107.23) (end 135.865 102.593) (width 0.2) (layer "F.Cu") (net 9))
 (segment (start 134.025 90.085) (end 135.29 88.82) (width 0.2) (layer "F.Cu") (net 9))
 (segment (start 133.705 107.23) (end 133.705 102.973) (width 0.2) (layer "F.Cu") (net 7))
 (segment (start 132.755 88.815) (end 132.75 88.81) (width 0.2) (layer "F.Cu") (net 7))
 (segment (start 132.75 97.7) (end 131.485 96.435) (width 0.2) (layer "F.Cu") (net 7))
 (segment (start 131.485 90.085) (end 132.755 88.815) (width 0.2) (layer "F.Cu") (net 7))
 (segment (start 131.485 96.435) (end 131.485 90.085) (width 0.2) (layer "F.Cu") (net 7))
 (segment (start 132.75 102.018) (end 132.75 98.3) (width 0.2) (layer "F.Cu") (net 7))
 (segment (start 133.705 102.973) (end 132.75 102.018) (width 0.2) (layer "F.Cu") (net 7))
 (segment (start 132.75 88.81) (end 132.75 85.6) (width 0.2) (layer "F.Cu") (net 7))
 (segment (start 132.75 98.3) (end 132.75 97.7) (width 0.2) (layer "F.Cu") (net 7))
 (segment (start 150.53 97.7) (end 149.265 96.435) (width 0.2) (layer "F.Cu") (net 17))
 (segment (start 149.265 96.435) (end 149.265 90.085) (width 0.2) (layer "F.Cu") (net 17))
 (segment (start 150.535 88.815) (end 150.53 88.81) (width 0.2) (layer "F.Cu") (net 17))
 (segment (start 149.265 90.085) (end 150.535 88.815) (width 0.2) (layer "F.Cu") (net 17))
 (segment (start 150.53 98.3) (end 150.53 97.7) (width 0.2) (layer "F.Cu") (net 17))
 (segment (start 150.53 101.774) (end 150.53 98.3) (width 0.2) (layer "F.Cu") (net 17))
 (segment (start 148.825 107.23) (end 148.825 103.479) (width 0.2) (layer "F.Cu") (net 17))
 (segment (start 148.825 103.479) (end 150.53 101.774) (width 0.2) (layer "F.Cu") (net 17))
 (segment (start 150.53 88.81) (end 150.53 85.6) (width 0.2) (layer "F.Cu") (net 17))
 (segment (start 140.37 98.3) (end 140.37 97.7) (width 0.2) (layer "F.Cu") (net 13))
 (segment (start 140.37 88.81) (end 140.37 85.6) (width 0.2) (layer "F.Cu") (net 13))
 (segment (start 140.185 107.23) (end 140.185 98.485) (width 0.2) (layer "F.Cu") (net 13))
 (segment (start 140.185 98.485) (end 140.37 98.3) (width 0.2) (layer "F.Cu") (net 13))
 (segment (start 139.105 90.085) (end 140.375 88.815) (width 0.2) (layer "F.Cu") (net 13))
 (segment (start 140.375 88.815) (end 140.37 88.81) (width 0.2) (layer "F.Cu") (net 13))
 (segment (start 139.105 96.435) (end 139.105 90.085) (width 0.2) (layer "F.Cu") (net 13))
 (segment (start 140.37 97.7) (end 139.105 96.435) (width 0.2) (layer "F.Cu") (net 13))
 (segment (start 134.025 102.023) (end 134.025 97.035) (width 0.2) (layer "F.Cu") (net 8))
 (segment (start 134.025 84.335) (end 132.75 83.06) (width 0.2) (layer "F.Cu") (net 8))
 (segment (start 134.787 102.785) (end 134.025 102.023) (width 0.2) (layer "F.Cu") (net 8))
 (segment (start 134.025 97.035) (end 132.75 95.76) (width 0.2) (layer "F.Cu") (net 8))
 (segment (start 134.787 109.389) (end 134.787 102.785) (width 0.2) (layer "F.Cu") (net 8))
 (segment (start 134.025 88.815) (end 134.025 84.335) (width 0.2) (layer "F.Cu") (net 8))
 (segment (start 132.75 90.09) (end 134.025 88.815) (width 0.2) (layer "F.Cu") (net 8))
 (segment (start 132.75 95.76) (end 132.75 90.09) (width 0.2) (layer "F.Cu") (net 8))
 (segment (start 133.705 110.471) (end 134.787 109.389) (width 0.2) (layer "F.Cu") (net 8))
 (segment (start 133.705 111.52) (end 133.705 110.471) (width 0.2) (layer "F.Cu") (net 8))
 (segment (start 128.437 103.801) (end 126.519 101.883) (width 0.2) (layer "F.Cu") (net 2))
 (segment (start 126.519 101.883) (end 126.519 97.149) (width 0.2) (layer "F.Cu") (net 2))
 (segment (start 127.225 110.347) (end 128.437 109.135) (width 0.2) (layer "F.Cu") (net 2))
 (segment (start 126.519 97.149) (end 125.13 95.76) (width 0.2) (layer "F.Cu") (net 2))
 (segment (start 127.225 111.52) (end 127.225 110.347) (width 0.2) (layer "F.Cu") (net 2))
 (segment (start 128.437 109.135) (end 128.437 103.801) (width 0.2) (layer "F.Cu") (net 2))
 (segment (start 125.13 95.76) (end 125.13 90.095) (width 0.2) (layer "F.Cu") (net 2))
 (segment (start 125.13 90.095) (end 126.405 88.82) (width 0.2) (layer "F.Cu") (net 2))
 (segment (start 126.405 84.335) (end 125.13 83.06) (width 0.2) (layer "F.Cu") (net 2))
 (segment (start 126.405 88.82) (end 126.405 84.335) (width 0.2) (layer "F.Cu") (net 2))
 (segment (start 136.819 109.643) (end 135.865 110.597) (width 0.2) (layer "F.Cu") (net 10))
 (segment (start 136.819 102.531) (end 136.819 109.643) (width 0.2) (layer "F.Cu") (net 10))
 (segment (start 135.29 95.76) (end 135.29 90.09) (width 0.2) (layer "F.Cu") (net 10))
 (segment (start 136.565 88.815) (end 136.565 84.335) (width 0.2) (layer "F.Cu") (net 10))
 (segment (start 135.29 90.09) (end 136.565 88.815) (width 0.2) (layer "F.Cu") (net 10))
 (segment (start 136.441 96.911) (end 136.441 102.153) (width 0.2) (layer "F.Cu") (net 10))
 (segment (start 136.565 84.335) (end 135.29 83.06) (width 0.2) (layer "F.Cu") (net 10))
 (segment (start 135.865 110.597) (end 135.865 111.52) (width 0.2) (layer "F.Cu") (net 10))
 (segment (start 136.441 102.153) (end 136.819 102.531) (width 0.2) (layer "F.Cu") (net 10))
 (segment (start 135.29 95.76) (end 136.441 96.911) (width 0.2) (layer "F.Cu") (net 10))
 (segment (start 157.515 115.485) (end 162.5 110.5) (width 1) (layer "F.Cu") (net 18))
 (segment (start 150.985 107.23) (end 150.985 103.605) (width 0.2) (layer "F.Cu") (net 18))
 (segment (start 153.07 97.7) (end 153.07 98.3) (width 0.2) (layer "F.Cu") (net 18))
 (segment (start 115.71 110.51) (end 120.685 115.485) (width 1) (layer "F.Cu") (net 18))
 (segment (start 153.07 101.52) (end 153.07 98.3) (width 0.2) (layer "F.Cu") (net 18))
 (segment (start 153.07 85.6) (end 153.07 88.82) (width 0.2) (layer "F.Cu") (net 18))
 (segment (start 162.5 110.5) (end 162.5 101.542) (width 1) (layer "F.Cu") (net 18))
 (segment (start 153.07 88.82) (end 151.805 90.085) (width 0.2) (layer "F.Cu") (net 18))
 (segment (start 162.5 101.542) (end 160.695 99.737) (width 1) (layer "F.Cu") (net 18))
 (segment (start 160.1 98.3) (end 160.695 97.705) (width 1) (layer "F.Cu") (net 18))
 (segment (start 153.07 98.3) (end 155.361 98.3) (width 1) (layer "F.Cu") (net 18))
 (segment (start 155.361 98.3) (end 160.1 98.3) (width 1) (layer "F.Cu") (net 18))
 (segment (start 150.985 103.605) (end 153.07 101.52) (width 0.2) (layer "F.Cu") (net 18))
 (segment (start 160.695 99.737) (end 160.695 97.705) (width 1) (layer "F.Cu") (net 18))
 (segment (start 120.685 115.485) (end 157.515 115.485) (width 1) (layer "F.Cu") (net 18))
 (segment (start 151.805 96.435) (end 153.07 97.7) (width 0.2) (layer "F.Cu") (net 18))
 (segment (start 151.805 90.085) (end 151.805 96.435) (width 0.2) (layer "F.Cu") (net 18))
 (segment (start 129.385 111.52) (end 129.385 110.219) (width 0.2) (layer "F.Cu") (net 4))
 (segment (start 129.385 110.219) (end 130.469 109.135) (width 0.2) (layer "F.Cu") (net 4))
 (segment (start 128.945 88.815) (end 128.945 84.335) (width 0.2) (layer "F.Cu") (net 4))
 (segment (start 128.945 101.769) (end 128.945 97.035) (width 0.2) (layer "F.Cu") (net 4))
 (segment (start 130.469 103.293) (end 128.945 101.769) (width 0.2) (layer "F.Cu") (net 4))
 (segment (start 128.945 84.335) (end 127.67 83.06) (width 0.2) (layer "F.Cu") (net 4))
 (segment (start 127.67 90.09) (end 128.945 88.815) (width 0.2) (layer "F.Cu") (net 4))
 (segment (start 128.945 97.035) (end 127.67 95.76) (width 0.2) (layer "F.Cu") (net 4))
 (segment (start 127.67 95.76) (end 127.67 90.09) (width 0.2) (layer "F.Cu") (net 4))
 (segment (start 130.469 109.135) (end 130.469 103.293) (width 0.2) (layer "F.Cu") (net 4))
 (segment (start 136.565 96.435) (end 136.565 90.085) (width 0.2) (layer "F.Cu") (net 11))
 (segment (start 137.83 88.81) (end 137.83 85.6) (width 0.2) (layer "F.Cu") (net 11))
 (segment (start 137.83 98.3) (end 137.83 97.7) (width 0.2) (layer "F.Cu") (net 11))
 (segment (start 137.83 102.018) (end 137.83 98.3) (width 0.2) (layer "F.Cu") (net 11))
 (segment (start 137.835 88.815) (end 137.83 88.81) (width 0.2) (layer "F.Cu") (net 11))
 (segment (start 138.025 107.23) (end 138.025 102.213) (width 0.2) (layer "F.Cu") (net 11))
 (segment (start 136.565 90.085) (end 137.835 88.815) (width 0.2) (layer "F.Cu") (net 11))
 (segment (start 137.83 97.7) (end 136.565 96.435) (width 0.2) (layer "F.Cu") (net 11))
 (segment (start 138.025 102.213) (end 137.83 102.018) (width 0.2) (layer "F.Cu") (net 11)))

